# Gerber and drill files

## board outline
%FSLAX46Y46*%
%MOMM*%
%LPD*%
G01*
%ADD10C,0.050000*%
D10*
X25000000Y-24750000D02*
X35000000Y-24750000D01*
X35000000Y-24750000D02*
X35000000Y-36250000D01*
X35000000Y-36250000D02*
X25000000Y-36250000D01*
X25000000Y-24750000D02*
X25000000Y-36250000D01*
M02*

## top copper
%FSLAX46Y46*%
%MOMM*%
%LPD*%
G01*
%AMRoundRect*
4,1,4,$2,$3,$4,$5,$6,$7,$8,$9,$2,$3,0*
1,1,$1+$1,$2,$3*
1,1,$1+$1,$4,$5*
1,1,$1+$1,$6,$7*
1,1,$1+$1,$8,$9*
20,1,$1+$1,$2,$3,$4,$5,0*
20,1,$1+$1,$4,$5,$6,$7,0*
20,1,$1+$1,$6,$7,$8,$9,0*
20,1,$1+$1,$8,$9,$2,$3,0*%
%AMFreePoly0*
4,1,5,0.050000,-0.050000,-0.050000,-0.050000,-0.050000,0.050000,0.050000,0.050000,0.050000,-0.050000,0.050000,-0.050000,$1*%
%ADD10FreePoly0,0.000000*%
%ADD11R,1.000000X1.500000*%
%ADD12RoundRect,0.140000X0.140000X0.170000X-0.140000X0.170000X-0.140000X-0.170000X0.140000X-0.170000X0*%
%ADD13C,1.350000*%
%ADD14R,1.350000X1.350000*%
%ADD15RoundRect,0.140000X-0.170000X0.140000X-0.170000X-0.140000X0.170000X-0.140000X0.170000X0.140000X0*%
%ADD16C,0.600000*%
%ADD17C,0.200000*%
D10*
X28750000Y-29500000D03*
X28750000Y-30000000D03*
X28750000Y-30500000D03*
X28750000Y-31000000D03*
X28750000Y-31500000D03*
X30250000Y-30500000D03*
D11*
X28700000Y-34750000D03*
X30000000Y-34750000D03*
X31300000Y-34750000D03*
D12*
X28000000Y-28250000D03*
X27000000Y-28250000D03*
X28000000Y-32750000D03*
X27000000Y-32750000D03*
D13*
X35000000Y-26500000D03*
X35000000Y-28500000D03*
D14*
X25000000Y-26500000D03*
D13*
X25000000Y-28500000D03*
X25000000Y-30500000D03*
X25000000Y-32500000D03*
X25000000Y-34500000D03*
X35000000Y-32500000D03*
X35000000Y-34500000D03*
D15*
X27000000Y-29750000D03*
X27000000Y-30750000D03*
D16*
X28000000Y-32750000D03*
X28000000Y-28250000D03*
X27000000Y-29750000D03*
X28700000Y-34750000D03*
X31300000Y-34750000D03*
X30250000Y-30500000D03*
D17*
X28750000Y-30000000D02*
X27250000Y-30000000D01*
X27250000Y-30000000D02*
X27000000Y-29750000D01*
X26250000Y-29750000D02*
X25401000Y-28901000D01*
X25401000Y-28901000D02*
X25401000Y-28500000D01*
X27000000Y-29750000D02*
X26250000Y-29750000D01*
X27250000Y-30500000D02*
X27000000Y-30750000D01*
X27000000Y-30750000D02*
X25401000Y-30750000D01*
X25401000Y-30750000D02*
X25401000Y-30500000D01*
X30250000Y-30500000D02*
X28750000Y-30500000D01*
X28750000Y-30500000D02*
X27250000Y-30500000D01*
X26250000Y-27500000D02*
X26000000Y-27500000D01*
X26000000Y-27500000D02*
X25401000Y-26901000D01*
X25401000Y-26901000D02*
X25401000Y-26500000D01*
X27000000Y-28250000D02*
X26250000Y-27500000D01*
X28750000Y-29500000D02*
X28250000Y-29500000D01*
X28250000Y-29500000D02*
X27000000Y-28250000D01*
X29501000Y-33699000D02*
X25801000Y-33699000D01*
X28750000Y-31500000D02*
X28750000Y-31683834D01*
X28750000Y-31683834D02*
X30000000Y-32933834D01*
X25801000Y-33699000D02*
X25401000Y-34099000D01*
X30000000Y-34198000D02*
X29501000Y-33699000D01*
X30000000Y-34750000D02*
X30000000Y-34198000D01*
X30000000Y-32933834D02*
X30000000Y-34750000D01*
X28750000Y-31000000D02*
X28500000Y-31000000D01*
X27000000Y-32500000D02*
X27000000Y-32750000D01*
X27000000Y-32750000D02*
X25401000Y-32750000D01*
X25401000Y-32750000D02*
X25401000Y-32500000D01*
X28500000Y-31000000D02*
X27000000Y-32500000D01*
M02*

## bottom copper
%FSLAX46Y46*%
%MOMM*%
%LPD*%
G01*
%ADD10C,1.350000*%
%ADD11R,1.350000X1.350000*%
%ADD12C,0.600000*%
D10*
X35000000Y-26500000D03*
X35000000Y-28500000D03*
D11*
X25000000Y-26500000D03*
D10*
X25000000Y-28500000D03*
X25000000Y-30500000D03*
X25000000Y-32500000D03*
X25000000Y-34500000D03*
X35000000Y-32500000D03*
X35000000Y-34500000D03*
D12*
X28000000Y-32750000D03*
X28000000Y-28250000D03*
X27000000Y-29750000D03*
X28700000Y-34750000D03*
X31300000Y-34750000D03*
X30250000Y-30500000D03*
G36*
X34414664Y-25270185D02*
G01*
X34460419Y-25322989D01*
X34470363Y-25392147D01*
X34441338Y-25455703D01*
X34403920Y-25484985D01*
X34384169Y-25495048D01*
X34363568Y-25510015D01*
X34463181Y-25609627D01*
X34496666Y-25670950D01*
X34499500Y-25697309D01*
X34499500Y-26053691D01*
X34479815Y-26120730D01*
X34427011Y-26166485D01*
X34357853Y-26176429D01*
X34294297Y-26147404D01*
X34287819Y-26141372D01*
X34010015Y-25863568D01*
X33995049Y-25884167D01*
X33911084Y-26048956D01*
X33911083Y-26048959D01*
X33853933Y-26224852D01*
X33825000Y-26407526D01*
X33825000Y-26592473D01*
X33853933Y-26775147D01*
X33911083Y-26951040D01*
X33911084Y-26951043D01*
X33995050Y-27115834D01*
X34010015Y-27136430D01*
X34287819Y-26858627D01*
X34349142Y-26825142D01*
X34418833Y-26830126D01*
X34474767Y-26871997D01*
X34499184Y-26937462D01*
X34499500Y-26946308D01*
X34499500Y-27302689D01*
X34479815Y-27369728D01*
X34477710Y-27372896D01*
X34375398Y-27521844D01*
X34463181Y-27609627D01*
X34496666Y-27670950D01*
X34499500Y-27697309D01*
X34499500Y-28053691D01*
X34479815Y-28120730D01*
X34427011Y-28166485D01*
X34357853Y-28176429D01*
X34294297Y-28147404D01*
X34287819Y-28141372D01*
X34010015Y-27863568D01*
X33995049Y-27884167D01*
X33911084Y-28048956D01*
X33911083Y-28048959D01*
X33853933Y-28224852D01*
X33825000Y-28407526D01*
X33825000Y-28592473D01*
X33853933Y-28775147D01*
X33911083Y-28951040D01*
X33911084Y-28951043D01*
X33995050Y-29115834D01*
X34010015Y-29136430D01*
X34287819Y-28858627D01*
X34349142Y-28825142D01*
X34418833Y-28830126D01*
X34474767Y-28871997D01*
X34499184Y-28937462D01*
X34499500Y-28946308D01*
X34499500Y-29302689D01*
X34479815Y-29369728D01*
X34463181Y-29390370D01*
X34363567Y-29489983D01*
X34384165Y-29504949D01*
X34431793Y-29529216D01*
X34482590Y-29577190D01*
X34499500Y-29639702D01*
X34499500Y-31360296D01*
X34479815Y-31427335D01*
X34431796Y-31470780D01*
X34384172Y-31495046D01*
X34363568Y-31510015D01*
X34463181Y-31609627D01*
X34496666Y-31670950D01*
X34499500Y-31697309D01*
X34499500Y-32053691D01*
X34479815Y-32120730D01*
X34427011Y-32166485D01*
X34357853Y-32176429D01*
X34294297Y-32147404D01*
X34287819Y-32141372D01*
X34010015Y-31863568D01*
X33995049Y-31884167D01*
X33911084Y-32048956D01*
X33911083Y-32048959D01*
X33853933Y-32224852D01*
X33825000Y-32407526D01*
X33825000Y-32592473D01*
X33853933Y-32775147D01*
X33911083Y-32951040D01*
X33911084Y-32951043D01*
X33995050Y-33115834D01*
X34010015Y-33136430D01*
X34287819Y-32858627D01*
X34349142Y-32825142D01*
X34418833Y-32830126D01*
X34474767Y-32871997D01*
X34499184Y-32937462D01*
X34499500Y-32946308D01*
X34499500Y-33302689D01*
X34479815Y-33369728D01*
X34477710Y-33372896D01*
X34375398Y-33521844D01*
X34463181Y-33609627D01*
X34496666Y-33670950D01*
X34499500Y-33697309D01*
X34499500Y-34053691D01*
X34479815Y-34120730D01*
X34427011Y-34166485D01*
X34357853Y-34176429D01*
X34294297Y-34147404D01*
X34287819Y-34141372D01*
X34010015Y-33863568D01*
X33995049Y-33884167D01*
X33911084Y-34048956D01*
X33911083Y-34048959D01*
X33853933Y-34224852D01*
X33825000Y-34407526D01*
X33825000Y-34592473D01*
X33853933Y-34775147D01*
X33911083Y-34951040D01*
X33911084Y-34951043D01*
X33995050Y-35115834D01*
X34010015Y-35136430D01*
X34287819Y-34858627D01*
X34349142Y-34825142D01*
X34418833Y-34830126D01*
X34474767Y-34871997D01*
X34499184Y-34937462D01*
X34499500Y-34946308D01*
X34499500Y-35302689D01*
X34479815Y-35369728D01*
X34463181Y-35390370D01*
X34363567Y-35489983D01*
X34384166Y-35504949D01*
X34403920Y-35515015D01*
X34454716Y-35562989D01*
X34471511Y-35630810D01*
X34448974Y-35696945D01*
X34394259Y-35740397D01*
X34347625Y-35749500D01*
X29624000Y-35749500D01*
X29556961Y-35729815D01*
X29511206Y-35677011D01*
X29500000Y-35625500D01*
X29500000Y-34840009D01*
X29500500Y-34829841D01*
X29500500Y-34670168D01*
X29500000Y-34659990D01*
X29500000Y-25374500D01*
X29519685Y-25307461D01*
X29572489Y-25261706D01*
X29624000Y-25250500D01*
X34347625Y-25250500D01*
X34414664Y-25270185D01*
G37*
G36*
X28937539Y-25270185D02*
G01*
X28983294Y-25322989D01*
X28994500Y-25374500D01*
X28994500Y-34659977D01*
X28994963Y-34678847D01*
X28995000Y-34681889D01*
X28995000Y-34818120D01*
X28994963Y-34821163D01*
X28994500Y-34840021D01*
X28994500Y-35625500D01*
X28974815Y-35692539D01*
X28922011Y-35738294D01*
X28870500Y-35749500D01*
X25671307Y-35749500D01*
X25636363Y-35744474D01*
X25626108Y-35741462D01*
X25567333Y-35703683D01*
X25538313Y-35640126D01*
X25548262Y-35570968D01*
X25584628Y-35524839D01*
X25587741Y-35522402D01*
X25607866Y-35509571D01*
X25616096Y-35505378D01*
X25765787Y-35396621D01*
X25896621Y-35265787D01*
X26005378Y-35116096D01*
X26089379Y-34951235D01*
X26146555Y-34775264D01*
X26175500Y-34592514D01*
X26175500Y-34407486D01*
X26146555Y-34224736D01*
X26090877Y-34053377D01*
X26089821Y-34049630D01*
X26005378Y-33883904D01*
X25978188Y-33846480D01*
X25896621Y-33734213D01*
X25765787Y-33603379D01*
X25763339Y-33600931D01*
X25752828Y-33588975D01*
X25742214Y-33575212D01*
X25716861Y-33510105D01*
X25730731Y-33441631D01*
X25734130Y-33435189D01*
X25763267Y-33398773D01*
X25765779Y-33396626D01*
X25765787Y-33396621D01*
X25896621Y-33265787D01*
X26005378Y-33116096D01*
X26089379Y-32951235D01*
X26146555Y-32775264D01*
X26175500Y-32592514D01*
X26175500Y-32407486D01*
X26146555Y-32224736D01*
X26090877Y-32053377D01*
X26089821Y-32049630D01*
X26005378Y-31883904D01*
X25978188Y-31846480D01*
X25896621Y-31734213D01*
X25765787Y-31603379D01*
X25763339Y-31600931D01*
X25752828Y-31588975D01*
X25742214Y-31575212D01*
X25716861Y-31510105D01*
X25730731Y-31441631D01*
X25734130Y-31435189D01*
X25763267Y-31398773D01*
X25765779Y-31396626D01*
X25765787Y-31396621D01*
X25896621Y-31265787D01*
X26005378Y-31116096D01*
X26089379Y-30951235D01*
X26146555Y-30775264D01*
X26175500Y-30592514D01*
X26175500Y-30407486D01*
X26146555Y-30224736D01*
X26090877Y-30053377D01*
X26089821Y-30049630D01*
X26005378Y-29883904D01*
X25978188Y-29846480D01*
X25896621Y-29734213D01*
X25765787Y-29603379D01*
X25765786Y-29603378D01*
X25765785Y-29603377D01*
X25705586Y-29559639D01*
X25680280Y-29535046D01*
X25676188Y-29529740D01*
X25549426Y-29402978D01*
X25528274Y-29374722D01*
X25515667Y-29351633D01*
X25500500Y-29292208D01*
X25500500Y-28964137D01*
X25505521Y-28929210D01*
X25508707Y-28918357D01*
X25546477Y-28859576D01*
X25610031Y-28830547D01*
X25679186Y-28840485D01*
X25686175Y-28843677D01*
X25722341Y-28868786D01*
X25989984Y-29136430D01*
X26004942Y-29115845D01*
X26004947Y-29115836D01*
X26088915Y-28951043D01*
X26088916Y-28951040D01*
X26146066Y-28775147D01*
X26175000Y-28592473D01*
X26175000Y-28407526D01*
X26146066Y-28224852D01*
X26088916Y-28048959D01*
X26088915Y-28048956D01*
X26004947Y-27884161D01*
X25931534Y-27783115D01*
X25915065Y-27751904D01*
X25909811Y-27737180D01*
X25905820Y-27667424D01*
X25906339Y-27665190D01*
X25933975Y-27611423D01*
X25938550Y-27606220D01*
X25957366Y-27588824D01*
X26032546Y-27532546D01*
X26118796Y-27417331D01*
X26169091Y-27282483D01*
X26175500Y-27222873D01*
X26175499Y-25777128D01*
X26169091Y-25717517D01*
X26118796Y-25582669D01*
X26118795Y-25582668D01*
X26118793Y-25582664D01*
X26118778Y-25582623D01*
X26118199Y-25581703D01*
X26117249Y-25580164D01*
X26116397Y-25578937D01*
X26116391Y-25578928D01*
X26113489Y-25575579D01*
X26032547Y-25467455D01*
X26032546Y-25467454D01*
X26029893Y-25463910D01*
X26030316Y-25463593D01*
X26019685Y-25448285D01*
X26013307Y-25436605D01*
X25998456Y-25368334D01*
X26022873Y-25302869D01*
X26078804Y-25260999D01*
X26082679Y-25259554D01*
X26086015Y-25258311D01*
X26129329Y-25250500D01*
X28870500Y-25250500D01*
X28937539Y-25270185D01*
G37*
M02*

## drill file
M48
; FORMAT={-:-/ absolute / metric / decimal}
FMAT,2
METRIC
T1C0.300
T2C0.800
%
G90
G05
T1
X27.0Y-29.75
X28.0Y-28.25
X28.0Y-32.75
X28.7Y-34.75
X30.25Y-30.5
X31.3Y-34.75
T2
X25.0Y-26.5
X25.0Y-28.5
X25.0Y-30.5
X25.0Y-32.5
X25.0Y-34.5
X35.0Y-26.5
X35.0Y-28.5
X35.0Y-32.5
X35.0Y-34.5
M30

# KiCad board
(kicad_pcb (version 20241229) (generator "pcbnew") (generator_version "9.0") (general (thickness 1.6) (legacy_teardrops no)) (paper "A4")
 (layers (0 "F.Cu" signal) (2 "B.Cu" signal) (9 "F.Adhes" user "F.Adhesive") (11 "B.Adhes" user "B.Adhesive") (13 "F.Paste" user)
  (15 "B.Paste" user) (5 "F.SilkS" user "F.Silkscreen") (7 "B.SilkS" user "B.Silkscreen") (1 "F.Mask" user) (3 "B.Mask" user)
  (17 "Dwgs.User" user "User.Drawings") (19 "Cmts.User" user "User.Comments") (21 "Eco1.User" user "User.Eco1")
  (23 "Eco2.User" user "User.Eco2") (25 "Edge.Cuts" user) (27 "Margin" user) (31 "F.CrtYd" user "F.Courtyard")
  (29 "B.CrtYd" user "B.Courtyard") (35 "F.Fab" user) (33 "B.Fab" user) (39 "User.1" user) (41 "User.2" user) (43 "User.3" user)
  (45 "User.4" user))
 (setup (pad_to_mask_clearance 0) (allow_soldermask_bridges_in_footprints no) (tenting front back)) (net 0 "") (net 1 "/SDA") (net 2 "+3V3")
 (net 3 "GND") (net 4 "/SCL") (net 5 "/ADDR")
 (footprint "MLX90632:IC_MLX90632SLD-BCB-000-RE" (layer "F.Cu") (at 30 30.5)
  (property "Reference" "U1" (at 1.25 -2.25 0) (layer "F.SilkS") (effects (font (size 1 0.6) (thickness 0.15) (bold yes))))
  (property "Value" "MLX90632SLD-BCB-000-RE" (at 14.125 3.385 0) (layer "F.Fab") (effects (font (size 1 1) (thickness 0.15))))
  (pad "1" smd custom (at -1.25 -1) (size 0.1 0.1) (layers "F.Cu") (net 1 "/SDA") (options (clearance outline) (anchor rect)) (primitives))
  (pad "2" smd custom (at -1.25 -0.5) (size 0.1 0.1) (layers "F.Cu") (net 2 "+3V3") (options (clearance outline) (anchor rect)) (primitives))
  (pad "3" smd custom (at -1.25 0) (size 0.1 0.1) (layers "F.Cu") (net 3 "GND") (options (clearance outline) (anchor rect)) (primitives))
  (pad "4" smd custom (at -1.25 0.5) (size 0.1 0.1) (layers "F.Cu") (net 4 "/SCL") (options (clearance outline) (anchor rect)) (primitives))
  (pad "5" smd custom (at -1.25 1) (size 0.1 0.1) (layers "F.Cu") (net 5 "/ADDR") (options (clearance outline) (anchor rect)) (primitives))
  (pad "6" smd custom (at 0.25 0) (size 0.1 0.1) (layers "F.Cu") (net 3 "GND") (options (clearance outline) (anchor rect)) (primitives)))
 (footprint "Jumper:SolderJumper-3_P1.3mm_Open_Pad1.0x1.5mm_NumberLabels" (layer "F.Cu") (at 30 34.75)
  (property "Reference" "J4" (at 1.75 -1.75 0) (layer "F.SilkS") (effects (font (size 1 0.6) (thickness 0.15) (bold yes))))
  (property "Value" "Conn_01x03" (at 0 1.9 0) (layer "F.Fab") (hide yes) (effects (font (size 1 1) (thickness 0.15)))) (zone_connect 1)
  (pad "1" smd rect (at -1.3 0) (size 1 1.5) (layers "F.Cu" "F.Mask") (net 2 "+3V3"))
  (pad "2" smd rect (at 0 0) (size 1 1.5) (layers "F.Cu" "F.Mask") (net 5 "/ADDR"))
  (pad "3" smd rect (at 1.3 0) (size 1 1.5) (layers "F.Cu" "F.Mask") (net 3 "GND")))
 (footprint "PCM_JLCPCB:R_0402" (layer "F.Cu") (at 27.5 28.25 180)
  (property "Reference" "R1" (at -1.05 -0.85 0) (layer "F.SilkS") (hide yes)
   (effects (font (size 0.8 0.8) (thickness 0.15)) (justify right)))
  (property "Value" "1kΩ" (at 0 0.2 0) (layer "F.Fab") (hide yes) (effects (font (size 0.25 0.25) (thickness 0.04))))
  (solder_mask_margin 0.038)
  (pad "1" smd roundrect (at -0.5 0 180) (size 0.56 0.62) (layers "F.Cu" "F.Mask" "F.Paste") (roundrect_rratio 0.25) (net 2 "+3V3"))
  (pad "2" smd roundrect (at 0.5 0 180) (size 0.56 0.62) (layers "F.Cu" "F.Mask" "F.Paste") (roundrect_rratio 0.25) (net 1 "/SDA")))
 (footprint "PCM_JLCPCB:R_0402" (layer "F.Cu") (at 27.5 32.75 180)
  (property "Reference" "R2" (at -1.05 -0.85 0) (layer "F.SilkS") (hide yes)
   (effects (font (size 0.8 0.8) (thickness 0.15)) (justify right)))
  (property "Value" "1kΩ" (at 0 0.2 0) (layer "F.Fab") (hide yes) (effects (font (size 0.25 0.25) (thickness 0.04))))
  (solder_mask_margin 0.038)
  (pad "1" smd roundrect (at -0.5 0 180) (size 0.56 0.62) (layers "F.Cu" "F.Mask" "F.Paste") (roundrect_rratio 0.25) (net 2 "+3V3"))
  (pad "2" smd roundrect (at 0.5 0 180) (size 0.56 0.62) (layers "F.Cu" "F.Mask" "F.Paste") (roundrect_rratio 0.25) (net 4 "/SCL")))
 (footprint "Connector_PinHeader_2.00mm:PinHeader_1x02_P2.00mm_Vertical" (layer "F.Cu") (at 35 26.5)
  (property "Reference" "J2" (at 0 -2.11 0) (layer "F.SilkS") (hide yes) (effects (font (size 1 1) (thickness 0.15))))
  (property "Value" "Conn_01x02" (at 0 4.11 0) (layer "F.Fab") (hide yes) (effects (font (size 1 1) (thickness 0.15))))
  (pad "1" thru_hole circle (at 0 0) (size 1.35 1.35) (drill 0.8) (layers "*.Cu" "*.Mask") (remove_unused_layers no) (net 3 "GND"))
  (pad "2" thru_hole circle (at 0 2) (size 1.35 1.35) (drill 0.8) (layers "*.Cu" "*.Mask") (remove_unused_layers no) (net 3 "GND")))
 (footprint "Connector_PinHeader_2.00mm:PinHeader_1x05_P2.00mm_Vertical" (layer "F.Cu") (at 25 26.5)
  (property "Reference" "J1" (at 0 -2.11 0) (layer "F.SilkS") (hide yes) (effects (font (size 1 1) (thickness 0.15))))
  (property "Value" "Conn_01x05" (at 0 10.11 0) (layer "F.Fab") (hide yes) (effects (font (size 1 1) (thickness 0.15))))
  (pad "1" thru_hole rect (at 0 0) (size 1.35 1.35) (drill 0.8) (layers "*.Cu" "*.Mask") (remove_unused_layers no) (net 1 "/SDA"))
  (pad "2" thru_hole circle (at 0 2) (size 1.35 1.35) (drill 0.8) (layers "*.Cu" "*.Mask") (remove_unused_layers no) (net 2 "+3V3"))
  (pad "3" thru_hole circle (at 0 4) (size 1.35 1.35) (drill 0.8) (layers "*.Cu" "*.Mask") (remove_unused_layers no) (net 3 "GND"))
  (pad "4" thru_hole circle (at 0 6) (size 1.35 1.35) (drill 0.8) (layers "*.Cu" "*.Mask") (remove_unused_layers no) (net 4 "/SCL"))
  (pad "5" thru_hole circle (at 0 8) (size 1.35 1.35) (drill 0.8) (layers "*.Cu" "*.Mask") (remove_unused_layers no) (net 5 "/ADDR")))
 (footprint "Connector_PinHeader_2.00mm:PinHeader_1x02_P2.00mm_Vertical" (layer "F.Cu") (at 35 32.5)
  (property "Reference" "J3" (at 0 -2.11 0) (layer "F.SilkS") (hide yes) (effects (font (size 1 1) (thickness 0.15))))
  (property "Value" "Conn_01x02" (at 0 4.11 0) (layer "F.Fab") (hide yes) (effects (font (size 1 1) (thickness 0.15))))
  (pad "1" thru_hole circle (at 0 0) (size 1.35 1.35) (drill 0.8) (layers "*.Cu" "*.Mask") (remove_unused_layers no) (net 3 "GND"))
  (pad "2" thru_hole circle (at 0 2) (size 1.35 1.35) (drill 0.8) (layers "*.Cu" "*.Mask") (remove_unused_layers no) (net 3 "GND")))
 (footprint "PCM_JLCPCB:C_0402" (layer "F.Cu") (at 27 30.25 -90)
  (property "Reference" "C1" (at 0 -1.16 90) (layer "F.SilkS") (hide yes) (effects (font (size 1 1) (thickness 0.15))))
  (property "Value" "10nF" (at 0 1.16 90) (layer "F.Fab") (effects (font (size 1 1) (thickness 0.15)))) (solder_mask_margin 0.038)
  (pad "1" smd roundrect (at -0.5 0 270) (size 0.56 0.62) (layers "F.Cu" "F.Mask" "F.Paste") (roundrect_rratio 0.25) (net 2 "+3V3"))
  (pad "2" smd roundrect (at 0.5 0 270) (size 0.56 0.62) (layers "F.Cu" "F.Mask" "F.Paste") (roundrect_rratio 0.25) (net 3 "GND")))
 (gr_line (start 25 24.75) (end 35 24.75) (stroke (width 0.05) (type default)) (layer "Edge.Cuts"))
 (gr_line (start 35 24.75) (end 35 36.25) (stroke (width 0.05) (type solid)) (layer "Edge.Cuts"))
 (gr_line (start 35 36.25) (end 25 36.25) (stroke (width 0.05) (type default)) (layer "Edge.Cuts"))
 (gr_line (start 25 24.75) (end 25 36.25) (stroke (width 0.05) (type solid)) (layer "Edge.Cuts"))
 (segment (start 28.75 30) (end 27.25 30) (width 0.2) (layer "F.Cu") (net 2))
 (segment (start 27.25 30) (end 27 29.75) (width 0.2) (layer "F.Cu") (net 2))
 (segment (start 26.25 29.75) (end 25.401 28.901) (width 0.2) (layer "F.Cu") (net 2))
 (segment (start 25.401 28.901) (end 25.401 28.5) (width 0.2) (layer "F.Cu") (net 2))
 (segment (start 27 29.75) (end 26.25 29.75) (width 0.2) (layer "F.Cu") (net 2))
 (via (at 28 32.75) (size 0.6) (drill 0.3) (layers "F.Cu" "B.Cu") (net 2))
 (via (at 28 28.25) (size 0.6) (drill 0.3) (layers "F.Cu" "B.Cu") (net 2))
 (via (at 27 29.75) (size 0.6) (drill 0.3) (layers "F.Cu" "B.Cu") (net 2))
 (via (at 28.7 34.75) (size 0.6) (drill 0.3) (layers "F.Cu" "B.Cu") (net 2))
 (segment (start 27.25 30.5) (end 27 30.75) (width 0.2) (layer "F.Cu") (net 3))
 (segment (start 27 30.75) (end 25.401 30.75) (width 0.2) (layer "F.Cu") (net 3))
 (segment (start 25.401 30.75) (end 25.401 30.5) (width 0.2) (layer "F.Cu") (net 3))
 (segment (start 30.25 30.5) (end 28.75 30.5) (width 0.2) (layer "F.Cu") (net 3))
 (segment (start 28.75 30.5) (end 27.25 30.5) (width 0.2) (layer "F.Cu") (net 3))
 (via (at 31.3 34.75) (size 0.6) (drill 0.3) (layers "F.Cu" "B.Cu") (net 3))
 (via (at 30.25 30.5) (size 0.6) (drill 0.3) (layers "F.Cu" "B.Cu") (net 3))
 (segment (start 26.25 27.5) (end 26 27.5) (width 0.2) (layer "F.Cu") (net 1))
 (segment (start 26 27.5) (end 25.401 26.901) (width 0.2) (layer "F.Cu") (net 1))
 (segment (start 25.401 26.901) (end 25.401 26.5) (width 0.2) (layer "F.Cu") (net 1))
 (segment (start 27 28.25) (end 26.25 27.5) (width 0.2) (layer "F.Cu") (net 1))
 (segment (start 28.75 29.5) (end 28.25 29.5) (width 0.2) (layer "F.Cu") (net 1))
 (segment (start 28.25 29.5) (end 27 28.25) (width 0.2) (layer "F.Cu") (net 1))
 (segment (start 29.501 33.699) (end 25.801 33.699) (width 0.2) (layer "F.Cu") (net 5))
 (segment (start 28.75 31.5) (end 28.75 31.683834) (width 0.2) (layer "F.Cu") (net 5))
 (segment (start 28.75 31.683834) (end 30 32.933834) (width 0.2) (layer "F.Cu") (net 5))
 (segment (start 25.801 33.699) (end 25.401 34.099) (width 0.2) (layer "F.Cu") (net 5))
 (segment (start 30 34.198) (end 29.501 33.699) (width 0.2) (layer "F.Cu") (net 5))
 (segment (start 30 34.75) (end 30 34.198) (width 0.2) (layer "F.Cu") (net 5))
 (segment (start 30 32.933834) (end 30 34.75) (width 0.2) (layer "F.Cu") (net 5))
 (segment (start 28.75 31) (end 28.5 31) (width 0.2) (layer "F.Cu") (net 4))
 (segment (start 27 32.5) (end 27 32.75) (width 0.2) (layer "F.Cu") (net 4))
 (segment (start 27 32.75) (end 25.401 32.75) (width 0.2) (layer "F.Cu") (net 4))
 (segment (start 25.401 32.75) (end 25.401 32.5) (width 0.2) (layer "F.Cu") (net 4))
 (segment (start 28.5 31) (end 27 32.5) (width 0.2) (layer "F.Cu") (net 4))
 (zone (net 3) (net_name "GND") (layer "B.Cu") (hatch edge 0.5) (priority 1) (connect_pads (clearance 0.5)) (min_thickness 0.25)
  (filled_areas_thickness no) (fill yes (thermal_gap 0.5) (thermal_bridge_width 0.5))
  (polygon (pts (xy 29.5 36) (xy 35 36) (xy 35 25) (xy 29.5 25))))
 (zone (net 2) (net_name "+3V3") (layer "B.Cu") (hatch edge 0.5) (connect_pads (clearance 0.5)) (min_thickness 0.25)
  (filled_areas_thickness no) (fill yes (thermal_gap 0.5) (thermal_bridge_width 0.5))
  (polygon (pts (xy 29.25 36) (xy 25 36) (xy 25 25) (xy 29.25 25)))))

